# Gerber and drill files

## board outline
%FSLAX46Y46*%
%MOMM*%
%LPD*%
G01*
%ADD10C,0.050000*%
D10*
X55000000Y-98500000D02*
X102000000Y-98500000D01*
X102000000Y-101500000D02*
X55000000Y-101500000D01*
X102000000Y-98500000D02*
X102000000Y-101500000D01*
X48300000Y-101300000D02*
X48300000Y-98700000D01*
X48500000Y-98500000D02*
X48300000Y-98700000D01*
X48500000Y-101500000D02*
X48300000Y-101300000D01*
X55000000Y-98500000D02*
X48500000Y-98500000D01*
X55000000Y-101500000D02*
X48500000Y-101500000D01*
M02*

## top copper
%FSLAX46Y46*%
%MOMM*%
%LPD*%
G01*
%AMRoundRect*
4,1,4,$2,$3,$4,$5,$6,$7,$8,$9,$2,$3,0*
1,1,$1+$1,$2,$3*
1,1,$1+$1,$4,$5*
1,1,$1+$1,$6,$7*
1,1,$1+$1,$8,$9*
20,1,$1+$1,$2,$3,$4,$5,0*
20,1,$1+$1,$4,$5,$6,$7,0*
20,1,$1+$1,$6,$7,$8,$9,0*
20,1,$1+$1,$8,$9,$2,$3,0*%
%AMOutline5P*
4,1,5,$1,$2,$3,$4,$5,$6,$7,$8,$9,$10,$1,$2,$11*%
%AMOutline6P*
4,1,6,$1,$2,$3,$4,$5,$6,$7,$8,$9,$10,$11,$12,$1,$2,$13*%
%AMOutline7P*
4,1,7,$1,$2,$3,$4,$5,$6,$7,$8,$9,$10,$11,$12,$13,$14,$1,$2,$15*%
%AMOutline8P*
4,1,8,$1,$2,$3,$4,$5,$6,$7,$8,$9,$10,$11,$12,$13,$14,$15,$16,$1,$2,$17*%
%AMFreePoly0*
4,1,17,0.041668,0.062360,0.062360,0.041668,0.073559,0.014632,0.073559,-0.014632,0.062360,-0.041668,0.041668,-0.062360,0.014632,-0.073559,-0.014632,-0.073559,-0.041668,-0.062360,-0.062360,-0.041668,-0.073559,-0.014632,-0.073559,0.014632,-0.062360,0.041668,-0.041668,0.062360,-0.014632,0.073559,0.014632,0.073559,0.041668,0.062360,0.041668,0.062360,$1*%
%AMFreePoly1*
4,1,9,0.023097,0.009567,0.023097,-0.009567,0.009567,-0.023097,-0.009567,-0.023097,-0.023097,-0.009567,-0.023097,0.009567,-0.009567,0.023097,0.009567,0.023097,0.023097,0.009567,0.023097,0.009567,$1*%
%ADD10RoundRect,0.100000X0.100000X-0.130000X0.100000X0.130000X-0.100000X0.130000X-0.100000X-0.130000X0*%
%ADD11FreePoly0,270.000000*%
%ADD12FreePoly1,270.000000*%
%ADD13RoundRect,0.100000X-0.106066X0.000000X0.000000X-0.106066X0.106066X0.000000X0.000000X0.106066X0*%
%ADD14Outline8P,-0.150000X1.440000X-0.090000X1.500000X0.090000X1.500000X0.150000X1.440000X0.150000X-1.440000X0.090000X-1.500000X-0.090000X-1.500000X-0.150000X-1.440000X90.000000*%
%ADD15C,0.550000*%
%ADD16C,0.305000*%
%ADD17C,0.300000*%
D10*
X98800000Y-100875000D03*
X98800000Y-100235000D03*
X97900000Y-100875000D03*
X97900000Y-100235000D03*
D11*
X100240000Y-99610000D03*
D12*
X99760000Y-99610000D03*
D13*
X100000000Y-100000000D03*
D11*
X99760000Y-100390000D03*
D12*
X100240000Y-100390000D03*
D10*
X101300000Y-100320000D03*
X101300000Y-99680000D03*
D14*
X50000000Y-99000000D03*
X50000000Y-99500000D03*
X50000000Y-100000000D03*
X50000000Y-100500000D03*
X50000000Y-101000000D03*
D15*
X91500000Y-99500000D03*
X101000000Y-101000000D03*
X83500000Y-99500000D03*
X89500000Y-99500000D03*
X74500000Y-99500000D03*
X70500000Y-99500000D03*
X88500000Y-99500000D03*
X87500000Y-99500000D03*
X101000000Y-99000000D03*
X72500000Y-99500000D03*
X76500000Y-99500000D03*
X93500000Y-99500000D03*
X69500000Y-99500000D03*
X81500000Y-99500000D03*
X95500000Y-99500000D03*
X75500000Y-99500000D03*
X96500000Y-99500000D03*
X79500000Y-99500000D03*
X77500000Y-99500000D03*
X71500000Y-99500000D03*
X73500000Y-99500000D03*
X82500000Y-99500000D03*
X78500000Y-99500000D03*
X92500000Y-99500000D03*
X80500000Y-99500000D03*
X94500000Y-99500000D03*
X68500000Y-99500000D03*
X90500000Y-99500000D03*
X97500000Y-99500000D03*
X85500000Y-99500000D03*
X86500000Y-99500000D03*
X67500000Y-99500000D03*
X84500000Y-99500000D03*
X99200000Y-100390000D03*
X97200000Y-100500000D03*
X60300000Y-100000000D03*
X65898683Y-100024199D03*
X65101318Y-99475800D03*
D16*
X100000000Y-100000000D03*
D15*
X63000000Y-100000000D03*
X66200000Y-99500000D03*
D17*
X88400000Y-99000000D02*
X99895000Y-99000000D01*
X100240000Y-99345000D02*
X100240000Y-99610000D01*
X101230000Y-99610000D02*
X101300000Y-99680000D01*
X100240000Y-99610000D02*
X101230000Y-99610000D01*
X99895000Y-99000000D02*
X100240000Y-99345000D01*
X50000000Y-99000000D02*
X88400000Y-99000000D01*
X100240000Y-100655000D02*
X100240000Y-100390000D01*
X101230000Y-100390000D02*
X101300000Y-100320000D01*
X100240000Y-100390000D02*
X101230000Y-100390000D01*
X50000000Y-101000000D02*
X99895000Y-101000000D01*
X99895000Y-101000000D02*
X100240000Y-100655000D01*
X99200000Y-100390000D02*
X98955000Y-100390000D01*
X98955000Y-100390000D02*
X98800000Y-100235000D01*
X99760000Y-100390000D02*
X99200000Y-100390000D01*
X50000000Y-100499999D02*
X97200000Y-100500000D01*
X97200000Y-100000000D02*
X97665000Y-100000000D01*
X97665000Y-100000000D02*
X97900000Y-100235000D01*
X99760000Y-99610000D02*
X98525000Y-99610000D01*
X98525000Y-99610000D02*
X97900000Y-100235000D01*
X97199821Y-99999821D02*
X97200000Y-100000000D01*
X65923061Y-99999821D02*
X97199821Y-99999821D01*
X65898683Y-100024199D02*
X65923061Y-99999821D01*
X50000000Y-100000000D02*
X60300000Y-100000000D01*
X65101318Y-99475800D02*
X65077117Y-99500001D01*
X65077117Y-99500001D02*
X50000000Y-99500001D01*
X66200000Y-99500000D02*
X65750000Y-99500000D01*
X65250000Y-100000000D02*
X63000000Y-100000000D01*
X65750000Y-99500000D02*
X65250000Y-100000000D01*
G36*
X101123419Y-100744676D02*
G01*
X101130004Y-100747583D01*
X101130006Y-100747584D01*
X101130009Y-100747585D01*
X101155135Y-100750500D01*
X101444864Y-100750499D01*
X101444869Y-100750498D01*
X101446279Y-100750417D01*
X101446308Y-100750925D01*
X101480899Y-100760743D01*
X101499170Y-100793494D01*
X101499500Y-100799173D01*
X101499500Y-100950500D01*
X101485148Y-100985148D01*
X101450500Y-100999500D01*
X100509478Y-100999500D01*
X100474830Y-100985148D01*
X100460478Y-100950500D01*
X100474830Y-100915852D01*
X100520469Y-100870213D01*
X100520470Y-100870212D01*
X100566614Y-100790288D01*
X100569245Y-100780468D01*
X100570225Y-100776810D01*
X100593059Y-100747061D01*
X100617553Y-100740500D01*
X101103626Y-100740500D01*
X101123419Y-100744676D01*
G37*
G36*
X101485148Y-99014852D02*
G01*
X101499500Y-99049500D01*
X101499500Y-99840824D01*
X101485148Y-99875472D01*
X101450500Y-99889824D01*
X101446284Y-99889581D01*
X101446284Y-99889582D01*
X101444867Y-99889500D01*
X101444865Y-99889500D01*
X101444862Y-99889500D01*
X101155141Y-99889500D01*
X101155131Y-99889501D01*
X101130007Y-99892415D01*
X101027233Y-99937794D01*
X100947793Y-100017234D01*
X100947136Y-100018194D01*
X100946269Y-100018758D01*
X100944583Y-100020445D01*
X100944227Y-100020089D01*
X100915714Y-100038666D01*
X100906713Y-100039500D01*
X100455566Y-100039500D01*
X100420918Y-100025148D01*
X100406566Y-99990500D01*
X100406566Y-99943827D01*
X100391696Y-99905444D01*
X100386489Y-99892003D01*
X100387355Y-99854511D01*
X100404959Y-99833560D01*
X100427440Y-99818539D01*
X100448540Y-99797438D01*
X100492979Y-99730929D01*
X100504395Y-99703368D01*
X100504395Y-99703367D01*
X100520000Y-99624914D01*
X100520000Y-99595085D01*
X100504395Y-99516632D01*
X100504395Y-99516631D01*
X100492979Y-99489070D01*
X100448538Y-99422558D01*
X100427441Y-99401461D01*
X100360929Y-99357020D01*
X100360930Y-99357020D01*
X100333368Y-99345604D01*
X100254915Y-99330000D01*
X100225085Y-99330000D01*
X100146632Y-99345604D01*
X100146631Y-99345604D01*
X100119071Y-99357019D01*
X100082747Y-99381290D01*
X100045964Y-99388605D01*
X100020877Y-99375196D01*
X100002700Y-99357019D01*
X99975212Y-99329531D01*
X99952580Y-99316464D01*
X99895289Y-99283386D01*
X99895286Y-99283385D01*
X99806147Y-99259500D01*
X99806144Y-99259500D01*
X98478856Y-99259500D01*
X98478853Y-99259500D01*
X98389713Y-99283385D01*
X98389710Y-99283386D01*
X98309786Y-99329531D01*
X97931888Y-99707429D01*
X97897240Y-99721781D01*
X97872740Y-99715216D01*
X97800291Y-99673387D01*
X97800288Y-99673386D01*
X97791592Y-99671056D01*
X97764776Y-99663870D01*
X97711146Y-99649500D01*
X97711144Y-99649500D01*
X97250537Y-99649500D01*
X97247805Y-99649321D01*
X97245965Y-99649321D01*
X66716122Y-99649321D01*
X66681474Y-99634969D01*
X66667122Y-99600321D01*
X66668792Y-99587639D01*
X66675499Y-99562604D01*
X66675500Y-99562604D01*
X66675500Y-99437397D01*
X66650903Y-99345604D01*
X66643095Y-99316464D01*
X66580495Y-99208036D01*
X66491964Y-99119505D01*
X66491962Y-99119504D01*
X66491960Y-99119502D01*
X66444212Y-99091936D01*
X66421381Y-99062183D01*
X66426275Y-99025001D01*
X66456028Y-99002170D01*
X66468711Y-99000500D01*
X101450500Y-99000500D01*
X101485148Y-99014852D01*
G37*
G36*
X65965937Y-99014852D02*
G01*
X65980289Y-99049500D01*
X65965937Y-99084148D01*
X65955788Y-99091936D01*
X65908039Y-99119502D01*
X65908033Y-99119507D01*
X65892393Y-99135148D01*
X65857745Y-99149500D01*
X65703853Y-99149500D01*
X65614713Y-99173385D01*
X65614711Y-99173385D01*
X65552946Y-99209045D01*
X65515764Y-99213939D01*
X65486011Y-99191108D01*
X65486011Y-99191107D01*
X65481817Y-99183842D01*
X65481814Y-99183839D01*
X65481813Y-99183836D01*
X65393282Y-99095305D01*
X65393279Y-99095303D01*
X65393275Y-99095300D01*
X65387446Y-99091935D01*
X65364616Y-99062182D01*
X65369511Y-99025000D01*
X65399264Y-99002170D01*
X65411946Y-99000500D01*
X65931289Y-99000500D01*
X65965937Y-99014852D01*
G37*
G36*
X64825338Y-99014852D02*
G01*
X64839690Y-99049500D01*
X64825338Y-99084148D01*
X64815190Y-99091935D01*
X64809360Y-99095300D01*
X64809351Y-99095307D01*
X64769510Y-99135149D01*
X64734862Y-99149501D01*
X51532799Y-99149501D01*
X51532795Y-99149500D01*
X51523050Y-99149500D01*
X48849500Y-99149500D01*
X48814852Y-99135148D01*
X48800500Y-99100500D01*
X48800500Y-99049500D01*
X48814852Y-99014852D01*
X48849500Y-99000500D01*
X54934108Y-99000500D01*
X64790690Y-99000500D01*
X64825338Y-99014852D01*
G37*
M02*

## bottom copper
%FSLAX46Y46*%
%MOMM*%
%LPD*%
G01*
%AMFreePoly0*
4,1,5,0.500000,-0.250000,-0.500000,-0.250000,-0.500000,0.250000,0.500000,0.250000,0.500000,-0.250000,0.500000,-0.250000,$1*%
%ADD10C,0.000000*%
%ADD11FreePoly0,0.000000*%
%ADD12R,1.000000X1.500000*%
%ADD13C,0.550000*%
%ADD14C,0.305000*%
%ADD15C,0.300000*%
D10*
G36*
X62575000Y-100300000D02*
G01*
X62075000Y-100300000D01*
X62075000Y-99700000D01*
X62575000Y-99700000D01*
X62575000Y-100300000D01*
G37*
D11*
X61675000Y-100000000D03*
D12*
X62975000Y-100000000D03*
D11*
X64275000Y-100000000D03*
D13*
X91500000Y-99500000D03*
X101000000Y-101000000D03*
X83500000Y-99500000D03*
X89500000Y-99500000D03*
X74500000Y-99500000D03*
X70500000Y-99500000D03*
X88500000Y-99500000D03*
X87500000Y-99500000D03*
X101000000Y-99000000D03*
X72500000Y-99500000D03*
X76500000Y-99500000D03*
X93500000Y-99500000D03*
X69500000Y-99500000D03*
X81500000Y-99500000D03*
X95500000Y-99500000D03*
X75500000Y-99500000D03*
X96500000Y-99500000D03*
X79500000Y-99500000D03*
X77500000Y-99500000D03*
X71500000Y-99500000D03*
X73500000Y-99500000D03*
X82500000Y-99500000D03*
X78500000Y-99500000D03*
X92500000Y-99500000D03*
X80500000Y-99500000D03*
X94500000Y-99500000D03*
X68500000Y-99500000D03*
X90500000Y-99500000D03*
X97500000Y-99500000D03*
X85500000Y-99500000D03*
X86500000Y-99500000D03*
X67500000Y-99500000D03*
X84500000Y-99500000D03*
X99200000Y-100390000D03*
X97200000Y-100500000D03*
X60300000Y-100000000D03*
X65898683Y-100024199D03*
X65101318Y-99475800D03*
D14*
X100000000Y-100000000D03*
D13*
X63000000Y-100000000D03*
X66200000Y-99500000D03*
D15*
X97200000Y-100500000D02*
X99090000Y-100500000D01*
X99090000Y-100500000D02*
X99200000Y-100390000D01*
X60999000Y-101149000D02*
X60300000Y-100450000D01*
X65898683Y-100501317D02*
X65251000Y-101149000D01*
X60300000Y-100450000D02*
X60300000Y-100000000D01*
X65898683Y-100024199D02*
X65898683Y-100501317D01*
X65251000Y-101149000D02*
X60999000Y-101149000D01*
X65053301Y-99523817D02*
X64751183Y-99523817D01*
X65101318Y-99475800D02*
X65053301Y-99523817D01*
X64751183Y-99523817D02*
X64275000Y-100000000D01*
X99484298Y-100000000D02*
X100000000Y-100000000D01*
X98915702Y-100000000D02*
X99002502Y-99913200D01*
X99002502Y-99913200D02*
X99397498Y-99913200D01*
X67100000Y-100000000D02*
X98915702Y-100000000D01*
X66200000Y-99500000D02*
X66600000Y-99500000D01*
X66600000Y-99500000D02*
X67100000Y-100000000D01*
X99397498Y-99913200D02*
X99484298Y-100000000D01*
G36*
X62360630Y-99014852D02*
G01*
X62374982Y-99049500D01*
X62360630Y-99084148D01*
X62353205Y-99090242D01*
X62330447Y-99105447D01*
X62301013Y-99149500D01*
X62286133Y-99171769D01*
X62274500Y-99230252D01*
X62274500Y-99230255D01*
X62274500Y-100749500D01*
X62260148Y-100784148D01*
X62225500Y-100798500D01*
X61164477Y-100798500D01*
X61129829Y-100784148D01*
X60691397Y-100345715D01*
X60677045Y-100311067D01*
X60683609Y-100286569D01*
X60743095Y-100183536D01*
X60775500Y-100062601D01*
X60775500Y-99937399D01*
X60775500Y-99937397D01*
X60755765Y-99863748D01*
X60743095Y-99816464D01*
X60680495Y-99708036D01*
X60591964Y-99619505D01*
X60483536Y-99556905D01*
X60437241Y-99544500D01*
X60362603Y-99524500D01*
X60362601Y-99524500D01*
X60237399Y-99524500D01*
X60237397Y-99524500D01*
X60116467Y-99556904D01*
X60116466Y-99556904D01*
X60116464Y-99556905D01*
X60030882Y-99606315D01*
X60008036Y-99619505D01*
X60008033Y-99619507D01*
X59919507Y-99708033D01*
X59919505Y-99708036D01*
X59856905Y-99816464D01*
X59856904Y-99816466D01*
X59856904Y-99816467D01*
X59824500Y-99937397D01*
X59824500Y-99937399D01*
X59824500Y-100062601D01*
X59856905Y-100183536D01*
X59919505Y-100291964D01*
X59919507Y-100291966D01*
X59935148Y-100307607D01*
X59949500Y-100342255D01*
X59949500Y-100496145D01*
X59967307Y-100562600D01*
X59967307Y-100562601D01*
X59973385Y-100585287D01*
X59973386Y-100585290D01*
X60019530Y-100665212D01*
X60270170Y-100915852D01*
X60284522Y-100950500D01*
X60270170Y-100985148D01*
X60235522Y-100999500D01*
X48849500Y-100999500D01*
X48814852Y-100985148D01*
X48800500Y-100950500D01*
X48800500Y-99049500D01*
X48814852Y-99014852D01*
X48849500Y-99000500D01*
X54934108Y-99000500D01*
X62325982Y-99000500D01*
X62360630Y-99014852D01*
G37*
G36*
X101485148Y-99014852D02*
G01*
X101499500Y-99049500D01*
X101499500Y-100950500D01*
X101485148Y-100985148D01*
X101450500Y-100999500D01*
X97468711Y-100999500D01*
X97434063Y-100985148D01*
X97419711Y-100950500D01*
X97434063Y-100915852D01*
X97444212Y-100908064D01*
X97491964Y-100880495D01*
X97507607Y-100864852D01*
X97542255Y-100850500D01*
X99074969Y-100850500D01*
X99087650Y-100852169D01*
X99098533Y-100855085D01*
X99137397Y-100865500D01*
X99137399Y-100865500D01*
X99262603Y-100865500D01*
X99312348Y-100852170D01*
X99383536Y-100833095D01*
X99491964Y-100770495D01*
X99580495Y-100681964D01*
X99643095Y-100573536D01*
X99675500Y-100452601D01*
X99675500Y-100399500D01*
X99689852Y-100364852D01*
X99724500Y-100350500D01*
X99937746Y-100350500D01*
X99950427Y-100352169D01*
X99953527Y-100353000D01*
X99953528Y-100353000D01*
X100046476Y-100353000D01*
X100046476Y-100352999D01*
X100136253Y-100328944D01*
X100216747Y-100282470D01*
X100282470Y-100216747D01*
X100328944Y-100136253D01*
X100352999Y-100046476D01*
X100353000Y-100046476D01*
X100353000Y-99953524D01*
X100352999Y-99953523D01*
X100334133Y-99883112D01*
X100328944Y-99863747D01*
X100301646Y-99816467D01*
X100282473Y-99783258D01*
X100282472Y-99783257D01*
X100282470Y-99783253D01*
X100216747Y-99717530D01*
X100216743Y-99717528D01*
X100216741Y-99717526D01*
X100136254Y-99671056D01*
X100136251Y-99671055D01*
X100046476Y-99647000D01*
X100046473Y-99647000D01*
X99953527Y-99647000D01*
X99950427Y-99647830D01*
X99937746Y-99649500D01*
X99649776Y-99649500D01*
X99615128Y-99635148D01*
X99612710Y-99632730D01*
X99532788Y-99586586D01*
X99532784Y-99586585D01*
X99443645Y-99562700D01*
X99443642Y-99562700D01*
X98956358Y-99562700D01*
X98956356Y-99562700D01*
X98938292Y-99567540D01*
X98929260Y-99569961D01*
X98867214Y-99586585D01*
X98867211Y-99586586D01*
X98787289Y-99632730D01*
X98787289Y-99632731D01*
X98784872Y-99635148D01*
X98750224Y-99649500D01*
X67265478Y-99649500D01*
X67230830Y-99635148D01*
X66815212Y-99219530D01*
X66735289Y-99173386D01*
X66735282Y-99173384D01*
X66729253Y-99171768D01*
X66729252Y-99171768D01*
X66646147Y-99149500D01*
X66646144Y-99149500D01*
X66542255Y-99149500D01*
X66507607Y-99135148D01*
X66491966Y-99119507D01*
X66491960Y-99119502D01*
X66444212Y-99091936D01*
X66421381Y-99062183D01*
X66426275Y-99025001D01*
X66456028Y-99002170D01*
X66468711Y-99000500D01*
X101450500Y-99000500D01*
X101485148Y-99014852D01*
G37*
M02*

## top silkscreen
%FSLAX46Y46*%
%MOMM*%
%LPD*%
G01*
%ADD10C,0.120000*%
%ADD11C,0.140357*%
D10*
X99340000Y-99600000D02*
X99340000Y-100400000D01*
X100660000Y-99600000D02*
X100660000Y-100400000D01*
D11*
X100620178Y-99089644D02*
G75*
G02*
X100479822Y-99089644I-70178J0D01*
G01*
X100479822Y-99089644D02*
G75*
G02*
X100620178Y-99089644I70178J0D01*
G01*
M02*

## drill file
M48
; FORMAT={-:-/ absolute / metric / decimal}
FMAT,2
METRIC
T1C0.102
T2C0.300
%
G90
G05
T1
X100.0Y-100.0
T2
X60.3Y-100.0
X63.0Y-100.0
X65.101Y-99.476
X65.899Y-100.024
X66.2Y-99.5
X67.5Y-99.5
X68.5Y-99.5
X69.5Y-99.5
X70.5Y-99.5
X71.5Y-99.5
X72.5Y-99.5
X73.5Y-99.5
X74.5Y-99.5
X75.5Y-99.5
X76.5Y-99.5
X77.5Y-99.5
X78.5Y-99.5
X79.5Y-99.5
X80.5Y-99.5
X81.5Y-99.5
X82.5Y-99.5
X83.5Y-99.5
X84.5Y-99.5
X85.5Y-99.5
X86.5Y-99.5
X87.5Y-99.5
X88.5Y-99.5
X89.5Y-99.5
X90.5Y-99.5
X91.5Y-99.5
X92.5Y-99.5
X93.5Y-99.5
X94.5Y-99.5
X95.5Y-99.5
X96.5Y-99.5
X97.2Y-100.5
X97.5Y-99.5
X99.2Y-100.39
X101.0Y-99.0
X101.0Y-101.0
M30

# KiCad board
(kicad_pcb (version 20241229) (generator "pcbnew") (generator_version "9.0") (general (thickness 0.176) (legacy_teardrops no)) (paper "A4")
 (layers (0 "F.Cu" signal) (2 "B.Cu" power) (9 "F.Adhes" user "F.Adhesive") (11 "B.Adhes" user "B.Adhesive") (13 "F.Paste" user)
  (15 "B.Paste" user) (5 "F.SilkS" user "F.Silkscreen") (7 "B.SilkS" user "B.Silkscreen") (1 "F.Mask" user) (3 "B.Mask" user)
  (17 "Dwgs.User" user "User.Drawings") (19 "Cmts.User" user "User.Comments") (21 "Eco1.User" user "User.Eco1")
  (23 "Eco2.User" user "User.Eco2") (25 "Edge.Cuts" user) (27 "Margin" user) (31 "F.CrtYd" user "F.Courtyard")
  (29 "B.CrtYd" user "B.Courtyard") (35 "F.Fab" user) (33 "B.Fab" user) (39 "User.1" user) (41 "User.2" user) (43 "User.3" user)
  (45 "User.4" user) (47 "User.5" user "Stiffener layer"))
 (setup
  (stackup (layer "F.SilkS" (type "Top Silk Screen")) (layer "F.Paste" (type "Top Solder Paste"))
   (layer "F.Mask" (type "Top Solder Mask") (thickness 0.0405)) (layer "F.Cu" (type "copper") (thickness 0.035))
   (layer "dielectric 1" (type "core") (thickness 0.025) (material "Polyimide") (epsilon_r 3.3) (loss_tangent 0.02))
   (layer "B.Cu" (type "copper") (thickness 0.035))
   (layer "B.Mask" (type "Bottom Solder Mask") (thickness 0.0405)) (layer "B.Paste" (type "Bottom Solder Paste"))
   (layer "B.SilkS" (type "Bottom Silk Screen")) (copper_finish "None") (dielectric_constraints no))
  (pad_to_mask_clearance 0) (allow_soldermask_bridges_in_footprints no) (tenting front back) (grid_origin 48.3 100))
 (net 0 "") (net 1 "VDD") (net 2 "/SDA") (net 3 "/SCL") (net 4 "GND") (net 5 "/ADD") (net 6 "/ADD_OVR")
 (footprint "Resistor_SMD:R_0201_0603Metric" (layer "F.Cu") (at 98.8 100.555 90)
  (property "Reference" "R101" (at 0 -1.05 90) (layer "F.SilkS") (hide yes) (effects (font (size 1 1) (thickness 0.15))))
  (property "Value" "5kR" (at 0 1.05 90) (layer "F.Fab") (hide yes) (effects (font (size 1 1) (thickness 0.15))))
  (pad "" smd roundrect (at -0.345 0 90) (size 0.318 0.36) (layers "F.Paste") (roundrect_rratio 0.25))
  (pad "" smd roundrect (at 0.345 0 90) (size 0.318 0.36) (layers "F.Paste") (roundrect_rratio 0.25))
  (pad "1" smd roundrect (at -0.32 0 90) (size 0.46 0.4) (layers "F.Cu" "F.Mask") (roundrect_rratio 0.25) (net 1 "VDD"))
  (pad "2" smd roundrect (at 0.32 0 90) (size 0.46 0.4) (layers "F.Cu" "F.Mask") (roundrect_rratio 0.25) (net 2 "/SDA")))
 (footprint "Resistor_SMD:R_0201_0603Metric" (layer "F.Cu") (at 97.9 100.555 90)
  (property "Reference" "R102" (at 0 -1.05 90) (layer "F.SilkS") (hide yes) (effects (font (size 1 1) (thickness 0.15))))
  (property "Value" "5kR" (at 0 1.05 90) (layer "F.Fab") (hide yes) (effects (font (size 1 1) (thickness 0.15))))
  (pad "" smd roundrect (at -0.345 0 90) (size 0.318 0.36) (layers "F.Paste") (roundrect_rratio 0.25))
  (pad "" smd roundrect (at 0.345 0 90) (size 0.318 0.36) (layers "F.Paste") (roundrect_rratio 0.25))
  (pad "1" smd roundrect (at -0.32 0 90) (size 0.46 0.4) (layers "F.Cu" "F.Mask") (roundrect_rratio 0.25) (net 1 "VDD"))
  (pad "2" smd roundrect (at 0.32 0 90) (size 0.46 0.4) (layers "F.Cu" "F.Mask") (roundrect_rratio 0.25) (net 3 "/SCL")))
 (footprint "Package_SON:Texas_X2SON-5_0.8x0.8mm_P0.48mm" (layer "F.Cu") (at 100 100 -90)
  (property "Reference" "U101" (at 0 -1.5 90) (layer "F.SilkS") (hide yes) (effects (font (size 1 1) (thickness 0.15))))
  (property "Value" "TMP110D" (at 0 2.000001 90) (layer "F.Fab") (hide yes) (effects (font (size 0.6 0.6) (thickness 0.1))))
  (fp_line (start -0.4 0.66) (end 0.4 0.66) (stroke (width 0.12) (type solid)) (layer "F.SilkS"))
  (fp_line (start -0.4 -0.66) (end 0.4 -0.66) (stroke (width 0.12) (type solid)) (layer "F.SilkS"))
  (fp_circle (center -0.910356 -0.55) (end -0.770356 -0.56) (stroke (width 0) (type solid)) (fill yes) (layer "F.SilkS"))
  (pad "" smd custom (at -0.39 -0.24 270) (size 0.15 0.15) (layers "F.Mask" "F.Paste") (zone_connect 0) (thermal_bridge_angle 90)
   (options (clearance outline) (anchor circle)) (primitives))
  (pad "" smd custom (at -0.39 0.24 270) (size 0.05 0.05) (layers "F.Mask" "F.Paste") (zone_connect 0) (thermal_bridge_angle 90)
   (options (clearance outline) (anchor circle)) (primitives))
  (pad "" smd custom (at 0.39 -0.24 270) (size 0.05 0.05) (layers "F.Mask" "F.Paste") (zone_connect 0) (thermal_bridge_angle 90)
   (options (clearance outline) (anchor circle)) (primitives))
  (pad "" smd custom (at 0.39 0.24 270) (size 0.15 0.15) (layers "F.Paste") (zone_connect 0) (thermal_bridge_angle 90)
   (options (clearance outline) (anchor circle)) (primitives))
  (pad "1" smd custom (at -0.39 -0.24 270) (size 0.15 0.15) (layers "F.Cu" "F.Mask") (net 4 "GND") (zone_connect 0)
   (thermal_bridge_angle 90) (options (clearance outline) (anchor circle)) (primitives))
  (pad "2" smd custom (at -0.39 0.24 270) (size 0.05 0.05) (layers "F.Cu" "F.Mask") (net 3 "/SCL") (zone_connect 0)
   (thermal_bridge_angle 90) (options (clearance outline) (anchor circle)) (primitives))
  (pad "3" smd roundrect (at 0 0 315) (size 0.35 0.35) (layers "F.Cu" "F.Mask" "F.Paste") (roundrect_rratio 0.2857142857) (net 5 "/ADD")
   (solder_mask_margin -0.05) (solder_paste_margin -0.055) (zone_connect 0))
  (pad "4" smd custom (at 0.39 0.24 270) (size 0.15 0.15) (layers "F.Cu" "F.Mask") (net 2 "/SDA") (zone_connect 0) (thermal_bridge_angle 90)
   (options (clearance outline) (anchor circle)) (primitives))
  (pad "5" smd custom (at 0.39 -0.24 270) (size 0.05 0.05) (layers "F.Cu" "F.Mask") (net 1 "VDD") (zone_connect 0) (thermal_bridge_angle 90)
   (options (clearance outline) (anchor circle)) (primitives)))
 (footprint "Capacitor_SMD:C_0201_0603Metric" (layer "F.Cu") (at 101.3 100 90)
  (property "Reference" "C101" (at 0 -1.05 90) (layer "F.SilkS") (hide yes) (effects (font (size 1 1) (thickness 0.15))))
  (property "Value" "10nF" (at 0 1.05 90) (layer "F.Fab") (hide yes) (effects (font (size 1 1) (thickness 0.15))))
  (pad "" smd roundrect (at -0.345 0 90) (size 0.318 0.36) (layers "F.Paste") (roundrect_rratio 0.25))
  (pad "" smd roundrect (at 0.345 0 90) (size 0.318 0.36) (layers "F.Paste") (roundrect_rratio 0.25))
  (pad "1" smd roundrect (at -0.32 0 90) (size 0.46 0.4) (layers "F.Cu" "F.Mask") (roundrect_rratio 0.25) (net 1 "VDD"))
  (pad "2" smd roundrect (at 0.32 0 90) (size 0.46 0.4) (layers "F.Cu" "F.Mask") (roundrect_rratio 0.25) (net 4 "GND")))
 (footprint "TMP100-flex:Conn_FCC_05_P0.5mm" (layer "F.Cu") (at 50 100 90)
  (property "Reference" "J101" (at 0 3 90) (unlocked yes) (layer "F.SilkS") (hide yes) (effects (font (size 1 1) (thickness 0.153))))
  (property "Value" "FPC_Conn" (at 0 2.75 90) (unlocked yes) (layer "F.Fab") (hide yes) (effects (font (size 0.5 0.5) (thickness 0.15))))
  (fp_line (start -1.3 -1.7) (end 1.3 -1.7) (stroke (width 0.05) (type default)) (layer "Edge.Cuts"))
  (fp_line (start 1.5 -1.5) (end 1.3 -1.7) (stroke (width 0.05) (type default)) (layer "Edge.Cuts"))
  (fp_line (start -1.5 -1.5) (end -1.3 -1.7) (stroke (width 0.05) (type default)) (layer "Edge.Cuts"))
  (fp_line (start 1.5 5) (end 1.5 -1.5) (stroke (width 0.05) (type default)) (layer "Edge.Cuts"))
  (fp_line (start -1.5 5) (end -1.5 -1.5) (stroke (width 0.05) (type default)) (layer "Edge.Cuts"))
  (pad "1" smd roundrect (at 1 0 90) (size 0.3 3) (layers "F.Cu" "F.Mask") (roundrect_rratio 0) (chamfer_ratio 0.2)
   (chamfer top_left top_right bottom_left bottom_right) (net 4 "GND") (thermal_bridge_angle 45))
  (pad "2" smd roundrect (at 0.5 0 90) (size 0.3 3) (layers "F.Cu" "F.Mask") (roundrect_rratio 0) (chamfer_ratio 0.2)
   (chamfer top_left top_right bottom_left bottom_right) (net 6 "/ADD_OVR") (thermal_bridge_angle 45))
  (pad "3" smd roundrect (at 0 0 90) (size 0.3 3) (layers "F.Cu" "F.Mask") (roundrect_rratio 0) (chamfer_ratio 0.2)
   (chamfer top_left top_right bottom_left bottom_right) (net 3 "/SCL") (thermal_bridge_angle 45))
  (pad "4" smd roundrect (at -0.5 0 90) (size 0.3 3) (layers "F.Cu" "F.Mask") (roundrect_rratio 0) (chamfer_ratio 0.2)
   (chamfer top_left top_right bottom_left bottom_right) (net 2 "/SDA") (thermal_bridge_angle 45))
  (pad "5" smd roundrect (at -1 0 90) (size 0.3 3) (layers "F.Cu" "F.Mask") (roundrect_rratio 0) (chamfer_ratio 0.2)
   (chamfer top_left top_right bottom_left bottom_right) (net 1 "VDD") (thermal_bridge_angle 45)))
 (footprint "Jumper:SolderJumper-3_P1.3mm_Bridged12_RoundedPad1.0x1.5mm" (layer "B.Cu") (at 62.975 100)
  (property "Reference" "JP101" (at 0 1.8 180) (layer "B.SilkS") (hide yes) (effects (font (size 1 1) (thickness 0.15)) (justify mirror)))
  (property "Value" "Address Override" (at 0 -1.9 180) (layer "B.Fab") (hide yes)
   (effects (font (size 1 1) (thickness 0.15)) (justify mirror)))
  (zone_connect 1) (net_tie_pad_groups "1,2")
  (fp_poly (pts (xy -0.9 0.3) (xy -0.4 0.3) (xy -0.4 -0.3) (xy -0.9 -0.3)) (stroke (width 0) (type solid)) (fill yes) (layer "B.Cu"))
  (pad "1" smd custom (at -1.3 0) (size 1 0.5) (layers "B.Cu" "B.Mask") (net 4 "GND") (zone_connect 2) (thermal_bridge_angle 45)
   (options (clearance outline) (anchor rect)) (primitives))
  (pad "2" smd rect (at 0 0) (size 1 1.5) (layers "B.Cu" "B.Mask") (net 5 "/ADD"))
  (pad "3" smd custom (at 1.3 0) (size 1 0.5) (layers "B.Cu" "B.Mask") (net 6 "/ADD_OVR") (zone_connect 2) (thermal_bridge_angle 45)
   (options (clearance outline) (anchor rect)) (primitives)))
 (gr_line (start 55 98.5) (end 102 98.5) (stroke (width 0.05) (type default)) (layer "Edge.Cuts"))
 (gr_line (start 102 101.5) (end 55 101.5) (stroke (width 0.05) (type default)) (layer "Edge.Cuts"))
 (gr_line (start 102 98.5) (end 102 101.5) (stroke (width 0.05) (type default)) (layer "Edge.Cuts"))
 (segment (start 88.4 99) (end 99.895 99) (width 0.3) (layer "F.Cu") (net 4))
 (segment (start 100.24 99.345) (end 100.24 99.61) (width 0.3) (layer "F.Cu") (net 4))
 (segment (start 101.23 99.61) (end 101.3 99.68) (width 0.3) (layer "F.Cu") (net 4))
 (segment (start 100.24 99.61) (end 101.23 99.61) (width 0.3) (layer "F.Cu") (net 4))
 (segment (start 99.895 99) (end 100.24 99.345) (width 0.3) (layer "F.Cu") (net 4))
 (segment (start 50 99) (end 88.4 99) (width 0.3) (layer "F.Cu") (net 4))
 (via (at 91.5 99.5) (size 0.55) (drill 0.3) (layers "F.Cu" "B.Cu") (free yes) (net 4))
 (via (at 101 101) (size 0.55) (drill 0.3) (layers "F.Cu" "B.Cu") (free yes) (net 4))
 (via (at 83.5 99.5) (size 0.55) (drill 0.3) (layers "F.Cu" "B.Cu") (free yes) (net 4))
 (via (at 89.5 99.5) (size 0.55) (drill 0.3) (layers "F.Cu" "B.Cu") (free yes) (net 4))
 (via (at 74.5 99.5) (size 0.55) (drill 0.3) (layers "F.Cu" "B.Cu") (free yes) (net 4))
 (via (at 70.5 99.5) (size 0.55) (drill 0.3) (layers "F.Cu" "B.Cu") (free yes) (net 4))
 (via (at 88.5 99.5) (size 0.55) (drill 0.3) (layers "F.Cu" "B.Cu") (free yes) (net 4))
 (via (at 87.5 99.5) (size 0.55) (drill 0.3) (layers "F.Cu" "B.Cu") (free yes) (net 4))
 (via (at 101 99) (size 0.55) (drill 0.3) (layers "F.Cu" "B.Cu") (free yes) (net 4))
 (via (at 72.5 99.5) (size 0.55) (drill 0.3) (layers "F.Cu" "B.Cu") (free yes) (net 4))
 (via (at 76.5 99.5) (size 0.55) (drill 0.3) (layers "F.Cu" "B.Cu") (free yes) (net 4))
 (via (at 93.5 99.5) (size 0.55) (drill 0.3) (layers "F.Cu" "B.Cu") (free yes) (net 4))
 (via (at 69.5 99.5) (size 0.55) (drill 0.3) (layers "F.Cu" "B.Cu") (free yes) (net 4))
 (via (at 81.5 99.5) (size 0.55) (drill 0.3) (layers "F.Cu" "B.Cu") (free yes) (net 4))
 (via (at 95.5 99.5) (size 0.55) (drill 0.3) (layers "F.Cu" "B.Cu") (free yes) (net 4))
 (via (at 75.5 99.5) (size 0.55) (drill 0.3) (layers "F.Cu" "B.Cu") (free yes) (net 4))
 (via (at 96.5 99.5) (size 0.55) (drill 0.3) (layers "F.Cu" "B.Cu") (free yes) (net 4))
 (via (at 79.5 99.5) (size 0.55) (drill 0.3) (layers "F.Cu" "B.Cu") (free yes) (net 4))
 (via (at 77.5 99.5) (size 0.55) (drill 0.3) (layers "F.Cu" "B.Cu") (free yes) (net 4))
 (via (at 71.5 99.5) (size 0.55) (drill 0.3) (layers "F.Cu" "B.Cu") (free yes) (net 4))
 (via (at 73.5 99.5) (size 0.55) (drill 0.3) (layers "F.Cu" "B.Cu") (free yes) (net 4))
 (via (at 82.5 99.5) (size 0.55) (drill 0.3) (layers "F.Cu" "B.Cu") (free yes) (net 4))
 (via (at 78.5 99.5) (size 0.55) (drill 0.3) (layers "F.Cu" "B.Cu") (free yes) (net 4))
 (via (at 92.5 99.5) (size 0.55) (drill 0.3) (layers "F.Cu" "B.Cu") (free yes) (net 4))
 (via (at 80.5 99.5) (size 0.55) (drill 0.3) (layers "F.Cu" "B.Cu") (free yes) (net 4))
 (via (at 94.5 99.5) (size 0.55) (drill 0.3) (layers "F.Cu" "B.Cu") (free yes) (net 4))
 (via (at 68.5 99.5) (size 0.55) (drill 0.3) (layers "F.Cu" "B.Cu") (free yes) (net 4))
 (via (at 90.5 99.5) (size 0.55) (drill 0.3) (layers "F.Cu" "B.Cu") (free yes) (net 4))
 (via (at 97.5 99.5) (size 0.55) (drill 0.3) (layers "F.Cu" "B.Cu") (free yes) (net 4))
 (via (at 85.5 99.5) (size 0.55) (drill 0.3) (layers "F.Cu" "B.Cu") (free yes) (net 4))
 (via (at 86.5 99.5) (size 0.55) (drill 0.3) (layers "F.Cu" "B.Cu") (free yes) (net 4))
 (via (at 67.5 99.5) (size 0.55) (drill 0.3) (layers "F.Cu" "B.Cu") (free yes) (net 4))
 (via (at 84.5 99.5) (size 0.55) (drill 0.3) (layers "F.Cu" "B.Cu") (free yes) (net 4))
 (segment (start 100.24 100.655) (end 100.24 100.39) (width 0.3) (layer "F.Cu") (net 1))
 (segment (start 101.23 100.39) (end 101.3 100.32) (width 0.3) (layer "F.Cu") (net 1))
 (segment (start 100.24 100.39) (end 101.23 100.39) (width 0.3) (layer "F.Cu") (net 1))
 (segment (start 50 101) (end 99.895 101) (width 0.3) (layer "F.Cu") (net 1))
 (segment (start 99.895 101) (end 100.24 100.655) (width 0.3) (layer "F.Cu") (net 1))
 (segment (start 99.2 100.39) (end 98.955 100.39) (width 0.3) (layer "F.Cu") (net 2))
 (segment (start 98.955 100.39) (end 98.8 100.235) (width 0.3) (layer "F.Cu") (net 2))
 (segment (start 99.76 100.39) (end 99.2 100.39) (width 0.3) (layer "F.Cu") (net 2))
 (segment (start 50 100.499999) (end 97.2 100.5) (width 0.3) (layer "F.Cu") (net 2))
 (via (at 99.2 100.39) (size 0.55) (drill 0.3) (layers "F.Cu" "B.Cu") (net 2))
 (via (at 97.2 100.5) (size 0.55) (drill 0.3) (layers "F.Cu" "B.Cu") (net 2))
 (segment (start 97.2 100.5) (end 99.09 100.5) (width 0.3) (layer "B.Cu") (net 2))
 (segment (start 99.09 100.5) (end 99.2 100.39) (width 0.3) (layer "B.Cu") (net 2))
 (segment (start 97.2 100) (end 97.665 100) (width 0.3) (layer "F.Cu") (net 3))
 (segment (start 97.665 100) (end 97.9 100.235) (width 0.3) (layer "F.Cu") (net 3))
 (segment (start 99.76 99.61) (end 98.525 99.61) (width 0.3) (layer "F.Cu") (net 3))
 (segment (start 98.525 99.61) (end 97.9 100.235) (width 0.3) (layer "F.Cu") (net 3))
 (segment (start 97.199821 99.999821) (end 97.2 100) (width 0.3) (layer "F.Cu") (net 3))
 (segment (start 65.923061 99.999821) (end 97.199821 99.999821) (width 0.3) (layer "F.Cu") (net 3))
 (segment (start 65.898683 100.024199) (end 65.923061 99.999821) (width 0.3) (layer "F.Cu") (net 3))
 (segment (start 50 100) (end 60.3 100) (width 0.3) (layer "F.Cu") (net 3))
 (via (at 60.3 100) (size 0.55) (drill 0.3) (layers "F.Cu" "B.Cu") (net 3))
 (via (at 65.898683 100.024199) (size 0.55) (drill 0.3) (layers "F.Cu" "B.Cu") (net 3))
 (segment (start 60.999 101.149) (end 60.3 100.45) (width 0.3) (layer "B.Cu") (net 3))
 (segment (start 65.898683 100.501317) (end 65.251 101.149) (width 0.3) (layer "B.Cu") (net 3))
 (segment (start 60.3 100.45) (end 60.3 100) (width 0.3) (layer "B.Cu") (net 3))
 (segment (start 65.898683 100.024199) (end 65.898683 100.501317) (width 0.3) (layer "B.Cu") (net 3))
 (segment (start 65.251 101.149) (end 60.999 101.149) (width 0.3) (layer "B.Cu") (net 3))
 (segment (start 65.101318 99.4758) (end 65.077117 99.500001) (width 0.3) (layer "F.Cu") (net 6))
 (segment (start 65.077117 99.500001) (end 50 99.500001) (width 0.3) (layer "F.Cu") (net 6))
 (via (at 65.101318 99.4758) (size 0.55) (drill 0.3) (layers "F.Cu" "B.Cu") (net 6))
 (segment (start 65.053301 99.523817) (end 64.751183 99.523817) (width 0.3) (layer "B.Cu") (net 6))
 (segment (start 65.101318 99.4758) (end 65.053301 99.523817) (width 0.3) (layer "B.Cu") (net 6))
 (segment (start 64.751183 99.523817) (end 64.275 100) (width 0.3) (layer "B.Cu") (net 6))
 (segment (start 66.2 99.5) (end 65.75 99.5) (width 0.3) (layer "F.Cu") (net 5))
 (segment (start 65.25 100) (end 63 100) (width 0.3) (layer "F.Cu") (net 5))
 (segment (start 65.75 99.5) (end 65.25 100) (width 0.3) (layer "F.Cu") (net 5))
 (via micro (at 100 100) (size 0.305) (drill 0.102) (layers "F.Cu" "B.Cu") (tenting none) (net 5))
 (via (at 63 100) (size 0.55) (drill 0.3) (layers "F.Cu" "B.Cu") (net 5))
 (via (at 66.2 99.5) (size 0.55) (drill 0.3) (layers "F.Cu" "B.Cu") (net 5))
 (segment (start 99.484298 100) (end 100 100) (width 0.3) (layer "B.Cu") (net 5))
 (segment (start 98.915702 100) (end 99.002502 99.9132) (width 0.3) (layer "B.Cu") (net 5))
 (segment (start 99.002502 99.9132) (end 99.397498 99.9132) (width 0.3) (layer "B.Cu") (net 5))
 (segment (start 67.1 100) (end 98.915702 100) (width 0.3) (layer "B.Cu") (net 5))
 (segment (start 66.2 99.5) (end 66.6 99.5) (width 0.3) (layer "B.Cu") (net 5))
 (segment (start 66.6 99.5) (end 67.1 100) (width 0.3) (layer "B.Cu") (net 5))
 (segment (start 99.397498 99.9132) (end 99.484298 100) (width 0.3) (layer "B.Cu") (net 5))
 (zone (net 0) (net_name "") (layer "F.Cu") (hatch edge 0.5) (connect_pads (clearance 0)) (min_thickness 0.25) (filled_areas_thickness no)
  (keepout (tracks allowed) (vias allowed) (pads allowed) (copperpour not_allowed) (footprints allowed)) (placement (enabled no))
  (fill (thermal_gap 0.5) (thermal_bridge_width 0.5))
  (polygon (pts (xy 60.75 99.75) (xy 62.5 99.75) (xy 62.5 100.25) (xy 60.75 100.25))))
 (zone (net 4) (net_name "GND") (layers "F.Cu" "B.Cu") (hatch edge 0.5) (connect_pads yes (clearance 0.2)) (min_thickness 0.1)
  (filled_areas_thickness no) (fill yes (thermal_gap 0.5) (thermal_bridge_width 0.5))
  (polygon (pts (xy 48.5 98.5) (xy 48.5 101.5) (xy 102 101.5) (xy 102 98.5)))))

